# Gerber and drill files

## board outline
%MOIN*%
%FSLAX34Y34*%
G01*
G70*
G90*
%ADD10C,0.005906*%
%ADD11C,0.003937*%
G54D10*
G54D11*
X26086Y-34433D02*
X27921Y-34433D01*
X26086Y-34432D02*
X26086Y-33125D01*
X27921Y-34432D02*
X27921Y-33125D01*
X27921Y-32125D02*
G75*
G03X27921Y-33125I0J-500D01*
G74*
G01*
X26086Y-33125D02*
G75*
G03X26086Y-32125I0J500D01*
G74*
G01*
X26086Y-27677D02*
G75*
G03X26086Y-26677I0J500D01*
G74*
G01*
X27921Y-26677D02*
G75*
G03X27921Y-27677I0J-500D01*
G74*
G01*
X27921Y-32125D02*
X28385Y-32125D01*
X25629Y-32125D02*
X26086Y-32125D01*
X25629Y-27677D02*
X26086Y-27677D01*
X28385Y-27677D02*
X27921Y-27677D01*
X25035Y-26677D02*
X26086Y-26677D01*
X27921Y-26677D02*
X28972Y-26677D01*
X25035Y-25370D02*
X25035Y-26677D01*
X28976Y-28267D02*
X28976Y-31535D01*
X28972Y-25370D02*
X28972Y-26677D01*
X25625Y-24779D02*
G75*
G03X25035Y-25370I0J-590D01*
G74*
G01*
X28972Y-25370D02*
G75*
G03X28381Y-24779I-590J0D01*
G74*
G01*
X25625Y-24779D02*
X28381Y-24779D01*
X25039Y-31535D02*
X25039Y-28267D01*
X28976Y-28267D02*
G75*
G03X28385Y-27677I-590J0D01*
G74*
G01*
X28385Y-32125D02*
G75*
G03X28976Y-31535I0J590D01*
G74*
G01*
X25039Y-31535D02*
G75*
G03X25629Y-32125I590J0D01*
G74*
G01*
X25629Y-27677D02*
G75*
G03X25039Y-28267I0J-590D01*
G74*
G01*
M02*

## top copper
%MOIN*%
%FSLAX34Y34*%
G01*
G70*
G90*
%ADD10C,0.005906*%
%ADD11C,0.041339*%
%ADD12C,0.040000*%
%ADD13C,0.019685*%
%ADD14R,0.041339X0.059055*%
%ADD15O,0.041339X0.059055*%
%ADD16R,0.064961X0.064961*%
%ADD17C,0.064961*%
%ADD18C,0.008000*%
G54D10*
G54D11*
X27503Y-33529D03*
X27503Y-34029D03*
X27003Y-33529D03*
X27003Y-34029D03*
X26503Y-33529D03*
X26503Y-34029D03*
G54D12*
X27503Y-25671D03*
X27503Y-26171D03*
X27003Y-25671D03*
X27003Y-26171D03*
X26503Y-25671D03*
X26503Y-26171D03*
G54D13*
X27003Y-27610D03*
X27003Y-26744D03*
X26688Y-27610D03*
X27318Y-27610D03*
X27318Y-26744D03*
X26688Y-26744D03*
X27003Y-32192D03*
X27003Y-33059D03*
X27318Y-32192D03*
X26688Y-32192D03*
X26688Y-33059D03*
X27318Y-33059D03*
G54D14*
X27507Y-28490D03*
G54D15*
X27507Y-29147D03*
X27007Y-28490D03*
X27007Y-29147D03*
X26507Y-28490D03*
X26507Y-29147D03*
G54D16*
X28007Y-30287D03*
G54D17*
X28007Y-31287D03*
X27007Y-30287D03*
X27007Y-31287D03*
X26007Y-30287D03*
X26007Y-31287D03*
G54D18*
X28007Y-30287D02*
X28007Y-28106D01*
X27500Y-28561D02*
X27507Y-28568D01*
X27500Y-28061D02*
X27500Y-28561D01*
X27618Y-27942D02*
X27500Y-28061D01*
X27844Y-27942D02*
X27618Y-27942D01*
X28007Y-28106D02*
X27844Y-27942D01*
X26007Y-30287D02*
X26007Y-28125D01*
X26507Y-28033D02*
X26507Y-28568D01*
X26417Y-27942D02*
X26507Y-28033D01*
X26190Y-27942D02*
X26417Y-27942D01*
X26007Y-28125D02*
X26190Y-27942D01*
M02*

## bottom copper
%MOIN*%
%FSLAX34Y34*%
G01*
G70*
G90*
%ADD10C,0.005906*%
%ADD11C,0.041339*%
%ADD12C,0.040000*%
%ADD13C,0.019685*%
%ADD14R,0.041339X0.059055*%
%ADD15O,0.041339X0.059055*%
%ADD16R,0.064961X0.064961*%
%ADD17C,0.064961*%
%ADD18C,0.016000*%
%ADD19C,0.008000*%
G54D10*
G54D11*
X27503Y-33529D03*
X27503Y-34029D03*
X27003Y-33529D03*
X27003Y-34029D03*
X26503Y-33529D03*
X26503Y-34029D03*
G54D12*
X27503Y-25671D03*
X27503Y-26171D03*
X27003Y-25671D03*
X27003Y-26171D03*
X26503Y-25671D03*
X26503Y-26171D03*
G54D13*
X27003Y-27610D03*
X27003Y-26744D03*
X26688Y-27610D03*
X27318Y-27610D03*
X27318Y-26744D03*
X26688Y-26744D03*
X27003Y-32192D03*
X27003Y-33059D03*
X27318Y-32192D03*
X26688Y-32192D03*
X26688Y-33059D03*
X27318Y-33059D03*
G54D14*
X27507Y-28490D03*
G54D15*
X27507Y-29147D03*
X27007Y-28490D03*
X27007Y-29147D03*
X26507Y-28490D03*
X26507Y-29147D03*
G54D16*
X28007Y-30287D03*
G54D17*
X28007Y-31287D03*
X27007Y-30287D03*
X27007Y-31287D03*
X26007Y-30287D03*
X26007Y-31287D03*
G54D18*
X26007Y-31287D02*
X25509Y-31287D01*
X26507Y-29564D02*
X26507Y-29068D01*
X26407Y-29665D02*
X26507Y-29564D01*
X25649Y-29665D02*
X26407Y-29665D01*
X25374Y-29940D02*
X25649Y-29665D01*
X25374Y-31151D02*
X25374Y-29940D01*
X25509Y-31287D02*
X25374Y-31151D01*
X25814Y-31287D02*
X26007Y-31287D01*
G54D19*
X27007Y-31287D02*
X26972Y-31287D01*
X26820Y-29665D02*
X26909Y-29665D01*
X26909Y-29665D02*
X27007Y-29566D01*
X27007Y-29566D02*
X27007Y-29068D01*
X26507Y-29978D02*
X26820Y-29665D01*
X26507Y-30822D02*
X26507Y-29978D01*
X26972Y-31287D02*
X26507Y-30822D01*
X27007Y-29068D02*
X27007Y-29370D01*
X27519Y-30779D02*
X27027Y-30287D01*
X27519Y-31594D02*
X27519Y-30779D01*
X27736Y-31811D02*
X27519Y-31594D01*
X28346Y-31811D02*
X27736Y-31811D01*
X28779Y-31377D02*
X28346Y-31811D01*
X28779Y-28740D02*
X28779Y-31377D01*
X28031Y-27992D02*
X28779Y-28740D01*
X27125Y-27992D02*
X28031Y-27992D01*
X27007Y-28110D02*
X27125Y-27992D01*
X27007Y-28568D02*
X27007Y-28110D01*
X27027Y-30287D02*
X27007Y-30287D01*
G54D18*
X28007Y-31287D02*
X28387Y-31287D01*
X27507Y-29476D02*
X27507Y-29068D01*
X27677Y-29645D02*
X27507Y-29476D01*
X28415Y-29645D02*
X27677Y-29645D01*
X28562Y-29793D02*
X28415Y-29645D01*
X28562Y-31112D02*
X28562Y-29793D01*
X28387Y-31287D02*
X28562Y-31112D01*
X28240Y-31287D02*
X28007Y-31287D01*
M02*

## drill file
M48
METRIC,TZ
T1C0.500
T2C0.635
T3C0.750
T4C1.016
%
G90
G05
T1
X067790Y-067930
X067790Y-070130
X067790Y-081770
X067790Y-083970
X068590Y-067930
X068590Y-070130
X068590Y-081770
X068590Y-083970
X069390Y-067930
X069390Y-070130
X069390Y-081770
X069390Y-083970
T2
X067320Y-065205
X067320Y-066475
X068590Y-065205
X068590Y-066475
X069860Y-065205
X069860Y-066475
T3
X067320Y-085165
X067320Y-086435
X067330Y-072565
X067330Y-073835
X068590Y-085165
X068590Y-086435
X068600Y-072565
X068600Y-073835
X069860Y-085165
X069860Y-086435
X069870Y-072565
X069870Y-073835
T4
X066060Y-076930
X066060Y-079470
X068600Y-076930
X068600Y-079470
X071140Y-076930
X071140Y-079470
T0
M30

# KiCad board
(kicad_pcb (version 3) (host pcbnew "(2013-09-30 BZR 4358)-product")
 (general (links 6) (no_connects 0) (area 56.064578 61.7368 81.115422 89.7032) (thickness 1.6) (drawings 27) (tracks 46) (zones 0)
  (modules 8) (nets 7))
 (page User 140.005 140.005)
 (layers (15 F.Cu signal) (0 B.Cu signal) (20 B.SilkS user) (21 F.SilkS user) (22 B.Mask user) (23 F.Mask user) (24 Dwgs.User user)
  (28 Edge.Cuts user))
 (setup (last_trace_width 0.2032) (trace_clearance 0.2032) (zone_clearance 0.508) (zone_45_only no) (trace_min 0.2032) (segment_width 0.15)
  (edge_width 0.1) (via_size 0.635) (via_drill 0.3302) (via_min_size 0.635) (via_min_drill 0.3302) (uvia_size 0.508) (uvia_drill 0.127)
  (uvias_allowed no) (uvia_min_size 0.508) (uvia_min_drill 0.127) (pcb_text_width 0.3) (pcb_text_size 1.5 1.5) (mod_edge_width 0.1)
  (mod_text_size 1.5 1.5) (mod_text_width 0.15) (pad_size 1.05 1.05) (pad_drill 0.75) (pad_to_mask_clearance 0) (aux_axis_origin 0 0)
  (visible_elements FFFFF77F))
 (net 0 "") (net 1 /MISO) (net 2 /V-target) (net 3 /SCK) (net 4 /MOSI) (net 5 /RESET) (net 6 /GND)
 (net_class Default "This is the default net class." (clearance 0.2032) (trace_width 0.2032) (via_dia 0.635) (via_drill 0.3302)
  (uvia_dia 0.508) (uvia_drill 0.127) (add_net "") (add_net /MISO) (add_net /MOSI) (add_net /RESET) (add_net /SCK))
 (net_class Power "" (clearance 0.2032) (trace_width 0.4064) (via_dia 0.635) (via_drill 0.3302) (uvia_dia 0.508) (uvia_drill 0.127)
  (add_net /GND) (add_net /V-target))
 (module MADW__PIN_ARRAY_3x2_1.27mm (layer F.Cu) (at 68.59 85.8 180) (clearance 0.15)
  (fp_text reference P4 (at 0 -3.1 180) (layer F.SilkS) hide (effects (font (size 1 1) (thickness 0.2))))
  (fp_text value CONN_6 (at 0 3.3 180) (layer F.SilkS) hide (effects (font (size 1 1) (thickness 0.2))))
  (pad 1 thru_hole circle (at -1.27 0.635 180) (size 1.05 1.05) (drill 0.75) (layers *.Cu *.Mask F.SilkS))
  (pad 2 thru_hole circle (at -1.27 -0.635 180) (size 1.05 1.05) (drill 0.75) (layers *.Cu *.Mask F.SilkS))
  (pad 3 thru_hole circle (at 0 0.635 180) (size 1.05 1.05) (drill 0.75) (layers *.Cu *.Mask F.SilkS))
  (pad 4 thru_hole circle (at 0 -0.635 180) (size 1.05 1.05) (drill 0.75) (layers *.Cu *.Mask F.SilkS))
  (pad 5 thru_hole circle (at 1.27 0.635 180) (size 1.05 1.05) (drill 0.75) (layers *.Cu *.Mask F.SilkS))
  (pad 6 thru_hole circle (at 1.27 -0.635 180) (size 1.05 1.05) (drill 0.75) (layers *.Cu *.Mask F.SilkS)))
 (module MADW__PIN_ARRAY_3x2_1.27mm (layer F.Cu) (at 68.59 65.84 180)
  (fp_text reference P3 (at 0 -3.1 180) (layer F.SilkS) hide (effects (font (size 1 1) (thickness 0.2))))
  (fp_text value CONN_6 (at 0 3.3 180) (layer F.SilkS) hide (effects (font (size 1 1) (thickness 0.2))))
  (pad 1 thru_hole circle (at -1.27 0.635 180) (size 1.016 1.016) (drill 0.635) (layers *.Cu *.Mask))
  (pad 2 thru_hole circle (at -1.27 -0.635 180) (size 1.016 1.016) (drill 0.635) (layers *.Cu *.Mask))
  (pad 3 thru_hole circle (at 0 0.635 180) (size 1.016 1.016) (drill 0.635) (layers *.Cu *.Mask))
  (pad 4 thru_hole circle (at 0 -0.635 180) (size 1.016 1.016) (drill 0.635) (layers *.Cu *.Mask))
  (pad 5 thru_hole circle (at 1.27 0.635 180) (size 1.016 1.016) (drill 0.635) (layers *.Cu *.Mask))
  (pad 6 thru_hole circle (at 1.27 -0.635 180) (size 1.016 1.016) (drill 0.635) (layers *.Cu *.Mask)))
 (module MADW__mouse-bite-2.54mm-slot (layer F.Cu) (at 68.59 69.03 180)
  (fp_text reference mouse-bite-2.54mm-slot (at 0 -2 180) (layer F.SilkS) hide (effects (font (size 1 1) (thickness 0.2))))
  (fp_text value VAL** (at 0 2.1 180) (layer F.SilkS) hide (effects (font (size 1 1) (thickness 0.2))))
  (pad "" thru_hole circle (at 0 -1.1 180) (size 0.5 0.5) (drill 0.5) (layers *.Cu))
  (pad "" thru_hole circle (at 0 1.1 180) (size 0.5 0.5) (drill 0.5) (layers *.Cu))
  (pad "" thru_hole circle (at 0.8 -1.1 180) (size 0.5 0.5) (drill 0.5) (layers *.Cu))
  (pad "" thru_hole circle (at -0.8 -1.1 180) (size 0.5 0.5) (drill 0.5) (layers *.Cu))
  (pad "" thru_hole circle (at -0.8 1.1 180) (size 0.5 0.5) (drill 0.5) (layers *.Cu))
  (pad "" thru_hole circle (at 0.8 1.1 180) (size 0.5 0.5) (drill 0.5) (layers *.Cu)))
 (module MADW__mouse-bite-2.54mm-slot (layer F.Cu) (at 68.59 82.87)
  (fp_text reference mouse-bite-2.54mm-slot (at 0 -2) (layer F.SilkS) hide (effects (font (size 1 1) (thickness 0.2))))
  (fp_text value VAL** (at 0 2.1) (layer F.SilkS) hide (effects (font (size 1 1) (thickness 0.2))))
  (pad "" thru_hole circle (at 0 -1.1) (size 0.5 0.5) (drill 0.5) (layers *.Cu))
  (pad "" thru_hole circle (at 0 1.1) (size 0.5 0.5) (drill 0.5) (layers *.Cu))
  (pad "" thru_hole circle (at 0.8 -1.1) (size 0.5 0.5) (drill 0.5) (layers *.Cu))
  (pad "" thru_hole circle (at -0.8 -1.1) (size 0.5 0.5) (drill 0.5) (layers *.Cu))
  (pad "" thru_hole circle (at -0.8 1.1) (size 0.5 0.5) (drill 0.5) (layers *.Cu))
  (pad "" thru_hole circle (at 0.8 1.1) (size 0.5 0.5) (drill 0.5) (layers *.Cu)))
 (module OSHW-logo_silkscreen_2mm (layer F.Cu) (at 65 74.1)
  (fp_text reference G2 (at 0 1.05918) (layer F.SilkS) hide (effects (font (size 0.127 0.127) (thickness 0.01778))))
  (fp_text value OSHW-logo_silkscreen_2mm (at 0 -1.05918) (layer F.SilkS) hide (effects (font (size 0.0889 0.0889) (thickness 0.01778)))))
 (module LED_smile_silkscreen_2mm (layer F.Cu) (at 65 71.7)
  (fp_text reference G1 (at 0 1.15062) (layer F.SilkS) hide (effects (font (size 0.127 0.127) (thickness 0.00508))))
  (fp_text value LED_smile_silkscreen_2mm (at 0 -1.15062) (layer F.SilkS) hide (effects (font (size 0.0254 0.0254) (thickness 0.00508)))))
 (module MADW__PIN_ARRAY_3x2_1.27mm (layer F.Cu) (at 68.6 73.2 180) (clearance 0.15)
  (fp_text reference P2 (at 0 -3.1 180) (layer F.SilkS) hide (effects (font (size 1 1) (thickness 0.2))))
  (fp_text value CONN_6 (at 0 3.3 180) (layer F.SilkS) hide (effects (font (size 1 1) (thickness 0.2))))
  (pad 1 thru_hole rect (at -1.27 0.635 180) (size 1.05 1.5) (drill 0.75 (offset 0 0.2)) (layers *.Cu *.Mask F.SilkS) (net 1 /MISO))
  (pad 2 thru_hole oval (at -1.27 -0.635 180) (size 1.05 1.5) (drill 0.75 (offset 0 -0.2)) (layers *.Cu *.Mask F.SilkS) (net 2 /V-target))
  (pad 3 thru_hole oval (at 0 0.635 180) (size 1.05 1.5) (drill 0.75 (offset 0 0.2)) (layers *.Cu *.Mask F.SilkS) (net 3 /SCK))
  (pad 4 thru_hole oval (at 0 -0.635 180) (size 1.05 1.5) (drill 0.75 (offset 0 -0.2)) (layers *.Cu *.Mask F.SilkS) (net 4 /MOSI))
  (pad 5 thru_hole oval (at 1.27 0.635 180) (size 1.05 1.5) (drill 0.75 (offset 0 0.2)) (layers *.Cu *.Mask F.SilkS) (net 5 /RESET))
  (pad 6 thru_hole oval (at 1.27 -0.635 180) (size 1.05 1.5) (drill 0.75 (offset 0 -0.2)) (layers *.Cu *.Mask F.SilkS) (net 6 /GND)))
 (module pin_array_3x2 (layer F.Cu) (at 68.6 78.2 180)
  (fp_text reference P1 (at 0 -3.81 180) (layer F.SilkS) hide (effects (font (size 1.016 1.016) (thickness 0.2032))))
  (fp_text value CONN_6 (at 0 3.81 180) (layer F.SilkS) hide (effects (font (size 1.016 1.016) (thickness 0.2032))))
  (pad 1 thru_hole rect (at -2.54 1.27 180) (size 1.65 1.65) (drill 1.016) (layers *.Cu *.Mask F.SilkS) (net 1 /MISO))
  (pad 2 thru_hole circle (at -2.54 -1.27 180) (size 1.65 1.65) (drill 1.016) (layers *.Cu *.Mask F.SilkS) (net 2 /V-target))
  (pad 3 thru_hole circle (at 0 1.27 180) (size 1.65 1.65) (drill 1.016) (layers *.Cu *.Mask F.SilkS) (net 3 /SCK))
  (pad 4 thru_hole circle (at 0 -1.27 180) (size 1.65 1.65) (drill 1.016) (layers *.Cu *.Mask F.SilkS) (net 4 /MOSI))
  (pad 5 thru_hole circle (at 2.54 1.27 180) (size 1.65 1.65) (drill 1.016) (layers *.Cu *.Mask F.SilkS) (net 5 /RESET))
  (pad 6 thru_hole circle (at 2.54 -1.27 180) (size 1.65 1.65) (drill 1.016) (layers *.Cu *.Mask F.SilkS) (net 6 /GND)))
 (gr_line (start 66.26 87.46) (end 70.92 87.46) (angle 90) (layer Edge.Cuts) (width 0.1))
 (gr_line (start 66.2595 87.4595) (end 66.2595 84.1395) (angle 90) (layer Edge.Cuts) (width 0.1))
 (gr_line (start 70.9195 87.4595) (end 70.9195 84.1395) (angle 90) (layer Edge.Cuts) (width 0.1))
 (gr_arc (start 70.92 82.87) (end 70.92 84.14) (angle 180) (layer Edge.Cuts) (width 0.1))
 (gr_arc (start 66.26 82.87) (end 66.26 81.6) (angle 180) (layer Edge.Cuts) (width 0.1))
 (gr_arc (start 66.26 69.03) (end 66.26 67.76) (angle 180) (layer Edge.Cuts) (width 0.1))
 (gr_arc (start 70.92 69.03) (end 70.92 70.3) (angle 180) (layer Edge.Cuts) (width 0.1))
 (gr_line (start 70.92 81.6) (end 72.1 81.6) (angle 90) (layer Edge.Cuts) (width 0.1))
 (gr_line (start 65.1 81.6) (end 66.26 81.6) (angle 90) (layer Edge.Cuts) (width 0.1))
 (gr_line (start 65.1 70.3) (end 66.26 70.3) (angle 90) (layer Edge.Cuts) (width 0.1))
 (gr_line (start 72.1 70.3) (end 70.92 70.3) (angle 90) (layer Edge.Cuts) (width 0.1))
 (gr_line (start 63.59 67.76) (end 66.26 67.76) (angle 90) (layer Edge.Cuts) (width 0.1))
 (gr_line (start 70.92 67.76) (end 73.59 67.76) (angle 90) (layer Edge.Cuts) (width 0.1))
 (gr_line (start 63.59 64.44) (end 63.59 67.76) (angle 90) (layer Edge.Cuts) (width 0.1))
 (gr_line (start 73.6 71.8) (end 73.6 80.1) (angle 90) (layer Edge.Cuts) (width 0.1))
 (gr_line (start 73.59 64.44) (end 73.59 67.76) (angle 90) (layer Edge.Cuts) (width 0.1))
 (gr_arc (start 65.09 64.44) (end 63.59 64.44) (angle 90) (layer Edge.Cuts) (width 0.1))
 (gr_arc (start 72.09 64.44) (end 72.09 62.94) (angle 90) (layer Edge.Cuts) (width 0.1))
 (gr_line (start 65.09 62.94) (end 72.09 62.94) (angle 90) (layer Edge.Cuts) (width 0.1))
 (gr_line (start 63.6 80.1) (end 63.6 71.8) (angle 90) (layer Edge.Cuts) (width 0.1))
 (gr_arc (start 72.1 71.8) (end 72.1 70.3) (angle 90) (layer Edge.Cuts) (width 0.1))
 (gr_arc (start 72.1 80.1) (end 73.6 80.1) (angle 90) (layer Edge.Cuts) (width 0.1))
 (gr_arc (start 65.1 80.1) (end 65.1 81.6) (angle 90) (layer Edge.Cuts) (width 0.1))
 (gr_arc (start 65.1 71.8) (end 63.6 71.8) (angle 90) (layer Edge.Cuts) (width 0.1))
 (segment (start 66.06 79.47) (end 64.795 79.47) (width 0.4064) (layer B.Cu) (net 6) (status 10))
 (segment (start 67.33 75.095) (end 67.33 73.835) (width 0.4064) (layer B.Cu) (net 6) (status 20))
 (segment (start 67.075 75.35) (end 67.33 75.095) (width 0.4064) (layer B.Cu) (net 6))
 (segment (start 65.15 75.35) (end 67.075 75.35) (width 0.4064) (layer B.Cu) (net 6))
 (segment (start 64.45 76.05) (end 65.15 75.35) (width 0.4064) (layer B.Cu) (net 6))
 (segment (start 64.45 79.125) (end 64.45 76.05) (width 0.4064) (layer B.Cu) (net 6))
 (segment (start 64.795 79.47) (end 64.45 79.125) (width 0.4064) (layer B.Cu) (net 6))
 (segment (start 65.57 79.47) (end 66.06 79.47) (width 0.4064) (layer B.Cu) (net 6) (status 30))
 (segment (start 71.14 76.93) (end 71.14 71.39) (width 0.2032) (layer F.Cu) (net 1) (status 10))
 (segment (start 69.85 72.545) (end 69.87 72.565) (width 0.2032) (layer F.Cu) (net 1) (status 30))
 (segment (start 69.85 71.275) (end 69.85 72.545) (width 0.2032) (layer F.Cu) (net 1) (status 20))
 (segment (start 70.15 70.975) (end 69.85 71.275) (width 0.2032) (layer F.Cu) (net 1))
 (segment (start 70.725 70.975) (end 70.15 70.975) (width 0.2032) (layer F.Cu) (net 1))
 (segment (start 71.14 71.39) (end 70.725 70.975) (width 0.2032) (layer F.Cu) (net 1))
 (segment (start 68.6 79.47) (end 68.51 79.47) (width 0.2032) (layer B.Cu) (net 4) (status 30))
 (segment (start 68.125 75.35) (end 68.35 75.35) (width 0.2032) (layer B.Cu) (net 4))
 (segment (start 68.35 75.35) (end 68.6 75.1) (width 0.2032) (layer B.Cu) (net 4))
 (segment (start 68.6 75.1) (end 68.6 73.835) (width 0.2032) (layer B.Cu) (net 4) (status 20))
 (segment (start 67.33 76.145) (end 68.125 75.35) (width 0.2032) (layer B.Cu) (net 4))
 (segment (start 67.33 78.29) (end 67.33 76.145) (width 0.2032) (layer B.Cu) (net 4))
 (segment (start 68.51 79.47) (end 67.33 78.29) (width 0.2032) (layer B.Cu) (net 4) (status 10))
 (segment (start 68.6 73.835) (end 68.6 74.6) (width 0.2032) (layer B.Cu) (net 4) (status 30))
 (segment (start 66.06 76.93) (end 66.06 71.44) (width 0.2032) (layer F.Cu) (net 5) (status 10))
 (segment (start 67.33 71.205) (end 67.33 72.565) (width 0.2032) (layer F.Cu) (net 5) (status 20))
 (segment (start 67.1 70.975) (end 67.33 71.205) (width 0.2032) (layer F.Cu) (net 5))
 (segment (start 66.525 70.975) (end 67.1 70.975) (width 0.2032) (layer F.Cu) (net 5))
 (segment (start 66.06 71.44) (end 66.525 70.975) (width 0.2032) (layer F.Cu) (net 5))
 (segment (start 69.9 78.18) (end 68.65 76.93) (width 0.2032) (layer B.Cu) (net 3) (status 20))
 (segment (start 69.9 80.25) (end 69.9 78.18) (width 0.2032) (layer B.Cu) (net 3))
 (segment (start 70.45 80.8) (end 69.9 80.25) (width 0.2032) (layer B.Cu) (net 3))
 (segment (start 72 80.8) (end 70.45 80.8) (width 0.2032) (layer B.Cu) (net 3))
 (segment (start 73.1 79.7) (end 72 80.8) (width 0.2032) (layer B.Cu) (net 3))
 (segment (start 73.1 73) (end 73.1 79.7) (width 0.2032) (layer B.Cu) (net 3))
 (segment (start 71.2 71.1) (end 73.1 73) (width 0.2032) (layer B.Cu) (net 3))
 (segment (start 68.9 71.1) (end 71.2 71.1) (width 0.2032) (layer B.Cu) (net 3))
 (segment (start 68.6 71.4) (end 68.9 71.1) (width 0.2032) (layer B.Cu) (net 3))
 (segment (start 68.6 72.565) (end 68.6 71.4) (width 0.2032) (layer B.Cu) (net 3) (status 10))
 (segment (start 68.65 76.93) (end 68.6 76.93) (width 0.2032) (layer B.Cu) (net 3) (status 30))
 (segment (start 71.14 79.47) (end 72.105 79.47) (width 0.4064) (layer B.Cu) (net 2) (status 10))
 (segment (start 69.87 74.87) (end 69.87 73.835) (width 0.4064) (layer B.Cu) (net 2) (status 20))
 (segment (start 70.3 75.3) (end 69.87 74.87) (width 0.4064) (layer B.Cu) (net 2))
 (segment (start 72.175 75.3) (end 70.3 75.3) (width 0.4064) (layer B.Cu) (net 2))
 (segment (start 72.55 75.675) (end 72.175 75.3) (width 0.4064) (layer B.Cu) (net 2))
 (segment (start 72.55 79.025) (end 72.55 75.675) (width 0.4064) (layer B.Cu) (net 2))
 (segment (start 72.105 79.47) (end 72.55 79.025) (width 0.4064) (layer B.Cu) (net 2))
 (segment (start 71.73 79.47) (end 71.14 79.47) (width 0.4064) (layer B.Cu) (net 2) (status 30)))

